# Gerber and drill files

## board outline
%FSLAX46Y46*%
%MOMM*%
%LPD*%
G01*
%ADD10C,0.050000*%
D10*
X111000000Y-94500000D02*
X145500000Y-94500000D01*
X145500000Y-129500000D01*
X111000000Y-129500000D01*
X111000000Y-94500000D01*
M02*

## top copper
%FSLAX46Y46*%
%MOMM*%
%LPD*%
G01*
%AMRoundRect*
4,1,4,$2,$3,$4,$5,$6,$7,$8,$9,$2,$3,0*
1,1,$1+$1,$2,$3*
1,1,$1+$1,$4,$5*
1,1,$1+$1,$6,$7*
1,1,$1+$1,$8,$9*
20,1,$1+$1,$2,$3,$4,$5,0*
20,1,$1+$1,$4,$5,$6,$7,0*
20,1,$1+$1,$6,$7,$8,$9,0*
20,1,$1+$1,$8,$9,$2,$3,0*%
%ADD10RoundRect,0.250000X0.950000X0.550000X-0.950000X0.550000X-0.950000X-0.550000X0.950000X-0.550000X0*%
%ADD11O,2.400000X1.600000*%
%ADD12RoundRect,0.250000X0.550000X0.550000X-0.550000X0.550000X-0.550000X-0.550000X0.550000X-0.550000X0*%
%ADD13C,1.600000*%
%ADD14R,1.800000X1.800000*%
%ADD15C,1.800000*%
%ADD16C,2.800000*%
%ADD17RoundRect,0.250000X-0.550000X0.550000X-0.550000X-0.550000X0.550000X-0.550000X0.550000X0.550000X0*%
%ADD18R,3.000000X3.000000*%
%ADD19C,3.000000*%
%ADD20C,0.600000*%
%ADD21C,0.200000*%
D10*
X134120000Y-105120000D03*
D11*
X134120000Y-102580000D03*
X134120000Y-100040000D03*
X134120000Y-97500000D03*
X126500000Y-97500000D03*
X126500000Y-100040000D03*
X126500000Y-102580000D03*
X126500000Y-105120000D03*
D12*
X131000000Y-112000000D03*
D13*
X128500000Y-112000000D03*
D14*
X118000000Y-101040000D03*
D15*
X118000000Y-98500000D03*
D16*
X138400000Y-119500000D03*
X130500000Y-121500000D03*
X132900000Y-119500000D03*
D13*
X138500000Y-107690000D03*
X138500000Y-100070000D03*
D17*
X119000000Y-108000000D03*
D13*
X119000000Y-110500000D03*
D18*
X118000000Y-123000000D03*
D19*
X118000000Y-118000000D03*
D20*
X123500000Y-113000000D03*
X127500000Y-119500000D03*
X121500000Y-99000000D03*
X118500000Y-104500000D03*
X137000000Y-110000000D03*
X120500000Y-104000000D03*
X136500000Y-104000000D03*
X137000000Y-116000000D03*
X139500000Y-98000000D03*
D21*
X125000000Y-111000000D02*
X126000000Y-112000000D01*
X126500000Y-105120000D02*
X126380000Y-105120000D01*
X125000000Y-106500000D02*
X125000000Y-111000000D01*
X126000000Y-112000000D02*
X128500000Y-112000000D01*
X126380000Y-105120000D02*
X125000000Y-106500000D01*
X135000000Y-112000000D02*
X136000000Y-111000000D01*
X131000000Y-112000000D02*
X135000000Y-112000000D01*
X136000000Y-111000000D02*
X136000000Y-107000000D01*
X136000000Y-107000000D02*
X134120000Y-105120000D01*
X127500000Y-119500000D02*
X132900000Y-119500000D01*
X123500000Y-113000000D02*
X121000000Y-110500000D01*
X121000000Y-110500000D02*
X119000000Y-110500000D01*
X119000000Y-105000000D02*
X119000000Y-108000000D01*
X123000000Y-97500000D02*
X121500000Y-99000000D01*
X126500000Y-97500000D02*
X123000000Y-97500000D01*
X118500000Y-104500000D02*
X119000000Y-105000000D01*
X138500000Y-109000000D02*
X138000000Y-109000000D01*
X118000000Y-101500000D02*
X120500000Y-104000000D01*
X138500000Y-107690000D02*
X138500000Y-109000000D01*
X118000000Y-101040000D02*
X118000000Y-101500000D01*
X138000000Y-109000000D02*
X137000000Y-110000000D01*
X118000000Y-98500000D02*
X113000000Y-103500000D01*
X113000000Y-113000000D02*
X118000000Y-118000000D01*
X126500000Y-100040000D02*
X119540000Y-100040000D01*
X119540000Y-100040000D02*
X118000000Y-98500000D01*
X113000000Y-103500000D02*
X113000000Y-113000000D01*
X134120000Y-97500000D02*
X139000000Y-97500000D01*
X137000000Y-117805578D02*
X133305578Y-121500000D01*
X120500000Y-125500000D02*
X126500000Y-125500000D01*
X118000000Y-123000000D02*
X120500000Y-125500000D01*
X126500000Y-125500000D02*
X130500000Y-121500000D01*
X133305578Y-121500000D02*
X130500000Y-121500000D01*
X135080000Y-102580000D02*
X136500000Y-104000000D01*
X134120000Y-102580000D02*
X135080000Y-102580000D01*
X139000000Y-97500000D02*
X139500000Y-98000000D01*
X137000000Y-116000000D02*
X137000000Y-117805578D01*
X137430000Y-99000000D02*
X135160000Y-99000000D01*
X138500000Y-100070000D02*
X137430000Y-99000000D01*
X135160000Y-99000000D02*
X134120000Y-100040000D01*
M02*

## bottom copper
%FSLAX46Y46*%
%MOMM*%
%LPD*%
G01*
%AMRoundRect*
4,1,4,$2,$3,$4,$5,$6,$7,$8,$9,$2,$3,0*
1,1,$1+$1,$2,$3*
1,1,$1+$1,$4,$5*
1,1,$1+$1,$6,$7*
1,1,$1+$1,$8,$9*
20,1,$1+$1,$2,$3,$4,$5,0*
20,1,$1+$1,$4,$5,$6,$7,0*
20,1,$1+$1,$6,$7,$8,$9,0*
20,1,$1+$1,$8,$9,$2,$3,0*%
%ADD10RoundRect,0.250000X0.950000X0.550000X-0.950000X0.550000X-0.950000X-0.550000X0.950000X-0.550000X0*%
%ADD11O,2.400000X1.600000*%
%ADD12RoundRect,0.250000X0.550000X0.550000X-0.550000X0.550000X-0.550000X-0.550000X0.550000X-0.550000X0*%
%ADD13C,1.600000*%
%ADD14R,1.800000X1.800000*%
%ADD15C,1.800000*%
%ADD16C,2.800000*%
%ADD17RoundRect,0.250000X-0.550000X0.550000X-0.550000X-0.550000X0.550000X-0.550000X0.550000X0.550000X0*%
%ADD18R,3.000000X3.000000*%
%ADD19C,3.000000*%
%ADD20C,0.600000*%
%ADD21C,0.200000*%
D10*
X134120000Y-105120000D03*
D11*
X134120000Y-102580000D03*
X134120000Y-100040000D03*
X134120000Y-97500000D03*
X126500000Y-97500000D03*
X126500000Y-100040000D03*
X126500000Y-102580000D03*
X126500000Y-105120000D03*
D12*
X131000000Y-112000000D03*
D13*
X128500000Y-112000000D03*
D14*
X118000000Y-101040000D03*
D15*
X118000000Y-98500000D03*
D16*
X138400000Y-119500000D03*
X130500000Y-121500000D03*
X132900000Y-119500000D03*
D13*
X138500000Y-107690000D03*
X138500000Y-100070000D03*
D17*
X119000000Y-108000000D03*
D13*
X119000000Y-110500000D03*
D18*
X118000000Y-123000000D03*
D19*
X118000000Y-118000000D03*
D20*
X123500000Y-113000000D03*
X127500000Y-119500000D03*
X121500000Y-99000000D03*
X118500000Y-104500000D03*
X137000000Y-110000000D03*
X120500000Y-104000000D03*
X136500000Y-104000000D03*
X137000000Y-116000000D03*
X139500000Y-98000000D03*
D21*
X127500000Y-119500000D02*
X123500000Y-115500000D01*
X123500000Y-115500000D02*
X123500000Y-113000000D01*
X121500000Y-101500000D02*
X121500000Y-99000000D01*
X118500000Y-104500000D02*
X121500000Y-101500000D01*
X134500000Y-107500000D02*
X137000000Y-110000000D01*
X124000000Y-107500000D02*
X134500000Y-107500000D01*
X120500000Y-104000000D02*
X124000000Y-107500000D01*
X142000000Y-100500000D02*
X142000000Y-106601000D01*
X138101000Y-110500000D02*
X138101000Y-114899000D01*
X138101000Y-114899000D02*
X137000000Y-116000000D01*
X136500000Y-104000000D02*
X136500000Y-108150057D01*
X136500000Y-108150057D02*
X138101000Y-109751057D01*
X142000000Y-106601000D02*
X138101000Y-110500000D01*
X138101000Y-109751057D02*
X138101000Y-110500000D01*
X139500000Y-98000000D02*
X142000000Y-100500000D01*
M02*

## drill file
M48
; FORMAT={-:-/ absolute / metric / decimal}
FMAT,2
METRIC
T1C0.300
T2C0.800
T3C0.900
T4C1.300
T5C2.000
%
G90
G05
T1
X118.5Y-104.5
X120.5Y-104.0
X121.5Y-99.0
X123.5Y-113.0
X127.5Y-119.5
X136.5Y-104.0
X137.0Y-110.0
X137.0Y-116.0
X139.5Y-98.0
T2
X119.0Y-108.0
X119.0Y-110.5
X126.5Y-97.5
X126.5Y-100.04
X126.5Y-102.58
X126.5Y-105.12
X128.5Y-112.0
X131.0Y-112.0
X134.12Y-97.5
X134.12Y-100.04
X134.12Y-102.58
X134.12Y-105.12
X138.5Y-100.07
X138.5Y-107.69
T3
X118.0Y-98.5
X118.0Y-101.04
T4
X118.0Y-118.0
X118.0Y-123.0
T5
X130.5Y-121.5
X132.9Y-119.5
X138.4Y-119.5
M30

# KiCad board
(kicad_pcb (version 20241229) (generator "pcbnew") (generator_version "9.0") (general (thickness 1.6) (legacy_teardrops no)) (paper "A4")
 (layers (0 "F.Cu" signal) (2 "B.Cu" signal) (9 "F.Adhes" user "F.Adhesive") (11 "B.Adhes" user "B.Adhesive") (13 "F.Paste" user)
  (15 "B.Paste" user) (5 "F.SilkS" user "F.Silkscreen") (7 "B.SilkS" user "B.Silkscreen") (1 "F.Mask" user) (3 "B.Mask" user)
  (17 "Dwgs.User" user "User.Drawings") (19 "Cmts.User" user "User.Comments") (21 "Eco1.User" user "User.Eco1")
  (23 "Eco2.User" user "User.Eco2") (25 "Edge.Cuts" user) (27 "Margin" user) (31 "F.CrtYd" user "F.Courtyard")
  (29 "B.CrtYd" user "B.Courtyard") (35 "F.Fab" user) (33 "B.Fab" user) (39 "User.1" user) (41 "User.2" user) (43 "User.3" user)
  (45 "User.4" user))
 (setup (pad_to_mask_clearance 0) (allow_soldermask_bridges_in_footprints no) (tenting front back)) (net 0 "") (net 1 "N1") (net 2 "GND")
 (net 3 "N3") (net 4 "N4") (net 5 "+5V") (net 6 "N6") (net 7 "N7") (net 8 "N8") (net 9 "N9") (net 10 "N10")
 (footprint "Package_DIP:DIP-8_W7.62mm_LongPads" (layer "F.Cu") (at 134.12 105.12 180)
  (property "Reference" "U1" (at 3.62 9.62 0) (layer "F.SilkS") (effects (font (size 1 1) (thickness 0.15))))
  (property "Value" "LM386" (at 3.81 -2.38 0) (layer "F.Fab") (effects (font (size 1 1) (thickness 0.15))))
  (pad "1" thru_hole roundrect (at 0 0 180) (size 2.4 1.6) (drill 0.8) (layers "*.Cu" "*.Mask") (remove_unused_layers no)
   (roundrect_rratio 0.15625) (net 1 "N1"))
  (pad "2" thru_hole oval (at 0 2.54 180) (size 2.4 1.6) (drill 0.8) (layers "*.Cu" "*.Mask") (remove_unused_layers no) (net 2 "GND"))
  (pad "3" thru_hole oval (at 0 5.08 180) (size 2.4 1.6) (drill 0.8) (layers "*.Cu" "*.Mask") (remove_unused_layers no) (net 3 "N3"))
  (pad "4" thru_hole oval (at 0 7.62 180) (size 2.4 1.6) (drill 0.8) (layers "*.Cu" "*.Mask") (remove_unused_layers no) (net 2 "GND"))
  (pad "5" thru_hole oval (at 7.62 7.62 180) (size 2.4 1.6) (drill 0.8) (layers "*.Cu" "*.Mask") (remove_unused_layers no) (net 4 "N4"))
  (pad "6" thru_hole oval (at 7.62 5.08 180) (size 2.4 1.6) (drill 0.8) (layers "*.Cu" "*.Mask") (remove_unused_layers no) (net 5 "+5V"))
  (pad "7" thru_hole oval (at 7.62 2.54 180) (size 2.4 1.6) (drill 0.8) (layers "*.Cu" "*.Mask") (remove_unused_layers no) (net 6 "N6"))
  (pad "8" thru_hole oval (at 7.62 0 180) (size 2.4 1.6) (drill 0.8) (layers "*.Cu" "*.Mask") (remove_unused_layers no) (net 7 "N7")))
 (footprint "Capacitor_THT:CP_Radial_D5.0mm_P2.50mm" (layer "F.Cu") (at 131 112 180)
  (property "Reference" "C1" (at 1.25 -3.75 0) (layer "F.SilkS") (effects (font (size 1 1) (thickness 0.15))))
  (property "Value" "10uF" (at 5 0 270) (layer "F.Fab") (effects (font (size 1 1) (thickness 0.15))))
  (pad "1" thru_hole roundrect (at 0 0 180) (size 1.6 1.6) (drill 0.8) (layers "*.Cu" "*.Mask") (remove_unused_layers no)
   (roundrect_rratio 0.15625) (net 1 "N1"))
  (pad "2" thru_hole circle (at 2.5 0 180) (size 1.6 1.6) (drill 0.8) (layers "*.Cu" "*.Mask") (remove_unused_layers no) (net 7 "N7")))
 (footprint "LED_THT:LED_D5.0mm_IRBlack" (layer "F.Cu") (at 118 101.04 90)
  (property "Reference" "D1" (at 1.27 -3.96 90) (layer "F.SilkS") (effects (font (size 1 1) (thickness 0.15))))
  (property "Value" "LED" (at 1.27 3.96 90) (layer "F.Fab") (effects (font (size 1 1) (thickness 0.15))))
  (pad "1" thru_hole rect (at 0 0 90) (size 1.8 1.8) (drill 0.9) (layers "*.Cu" "*.Mask") (remove_unused_layers no) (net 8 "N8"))
  (pad "2" thru_hole circle (at 2.54 0 90) (size 1.8 1.8) (drill 0.9) (layers "*.Cu" "*.Mask") (remove_unused_layers no) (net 5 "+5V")))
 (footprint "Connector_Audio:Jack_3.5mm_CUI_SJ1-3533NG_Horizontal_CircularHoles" (layer "F.Cu") (at 130.5 121.5 90)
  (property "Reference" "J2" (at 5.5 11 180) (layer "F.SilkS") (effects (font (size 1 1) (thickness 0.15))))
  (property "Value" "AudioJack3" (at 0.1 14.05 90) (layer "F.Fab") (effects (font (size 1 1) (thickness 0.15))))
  (pad "R" thru_hole circle (at 2 7.9 90) (size 2.8 2.8) (drill 2) (layers "*.Cu" "*.Mask") (remove_unused_layers no) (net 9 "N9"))
  (pad "S" thru_hole circle (at 0 0 90) (size 2.8 2.8) (drill 2) (layers "*.Cu" "*.Mask") (remove_unused_layers no) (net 2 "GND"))
  (pad "T" thru_hole circle (at 2 2.4 90) (size 2.8 2.8) (drill 2) (layers "*.Cu" "*.Mask") (remove_unused_layers no) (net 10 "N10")))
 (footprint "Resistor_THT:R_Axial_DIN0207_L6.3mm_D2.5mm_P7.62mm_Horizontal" (layer "F.Cu") (at 138.5 107.69 90)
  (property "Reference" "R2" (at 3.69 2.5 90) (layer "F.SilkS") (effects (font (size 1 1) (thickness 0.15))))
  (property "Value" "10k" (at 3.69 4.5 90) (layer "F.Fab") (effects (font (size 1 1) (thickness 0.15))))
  (pad "1" thru_hole circle (at 0 0 90) (size 1.6 1.6) (drill 0.8) (layers "*.Cu" "*.Mask") (remove_unused_layers no) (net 8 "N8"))
  (pad "2" thru_hole circle (at 7.62 0 90) (size 1.6 1.6) (drill 0.8) (layers "*.Cu" "*.Mask") (remove_unused_layers no) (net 3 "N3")))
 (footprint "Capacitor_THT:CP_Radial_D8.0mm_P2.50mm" (layer "F.Cu") (at 119 108 -90)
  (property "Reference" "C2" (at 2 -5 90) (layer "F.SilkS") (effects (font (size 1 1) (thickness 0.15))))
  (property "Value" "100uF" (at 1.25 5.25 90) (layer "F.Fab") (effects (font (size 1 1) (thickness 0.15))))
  (pad "1" thru_hole roundrect (at 0 0 270) (size 1.6 1.6) (drill 0.8) (layers "*.Cu" "*.Mask") (remove_unused_layers no)
   (roundrect_rratio 0.15625) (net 4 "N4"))
  (pad "2" thru_hole circle (at 2.5 0 270) (size 1.6 1.6) (drill 0.8) (layers "*.Cu" "*.Mask") (remove_unused_layers no) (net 10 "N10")))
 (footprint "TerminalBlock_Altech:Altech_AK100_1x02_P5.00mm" (layer "F.Cu") (at 118 123 90)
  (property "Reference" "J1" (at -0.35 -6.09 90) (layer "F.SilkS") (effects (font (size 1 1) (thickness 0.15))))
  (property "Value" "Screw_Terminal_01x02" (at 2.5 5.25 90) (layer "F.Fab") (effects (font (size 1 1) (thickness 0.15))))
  (pad "1" thru_hole rect (at 0 0 90) (size 3 3) (drill 1.3) (layers "*.Cu" "*.Mask") (remove_unused_layers no) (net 2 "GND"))
  (pad "2" thru_hole circle (at 5 0 90) (size 3 3) (drill 1.3) (layers "*.Cu" "*.Mask") (remove_unused_layers no) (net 5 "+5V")))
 (gr_rect (start 111 94.5) (end 145.5 129.5) (stroke (width 0.05) (type default)) (fill no) (layer "Edge.Cuts"))
 (segment (start 125 111) (end 126 112) (width 0.2) (layer "F.Cu") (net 7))
 (segment (start 126.5 105.12) (end 126.38 105.12) (width 0.2) (layer "F.Cu") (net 7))
 (segment (start 125 106.5) (end 125 111) (width 0.2) (layer "F.Cu") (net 7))
 (segment (start 126 112) (end 128.5 112) (width 0.2) (layer "F.Cu") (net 7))
 (segment (start 126.38 105.12) (end 125 106.5) (width 0.2) (layer "F.Cu") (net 7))
 (segment (start 135 112) (end 136 111) (width 0.2) (layer "F.Cu") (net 1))
 (segment (start 131 112) (end 135 112) (width 0.2) (layer "F.Cu") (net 1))
 (segment (start 136 111) (end 136 107) (width 0.2) (layer "F.Cu") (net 1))
 (segment (start 136 107) (end 134.12 105.12) (width 0.2) (layer "F.Cu") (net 1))
 (segment (start 127.5 119.5) (end 132.9 119.5) (width 0.2) (layer "F.Cu") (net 10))
 (segment (start 123.5 113) (end 121 110.5) (width 0.2) (layer "F.Cu") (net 10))
 (segment (start 121 110.5) (end 119 110.5) (width 0.2) (layer "F.Cu") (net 10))
 (via (at 123.5 113) (size 0.6) (drill 0.3) (layers "F.Cu" "B.Cu") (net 10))
 (via (at 127.5 119.5) (size 0.6) (drill 0.3) (layers "F.Cu" "B.Cu") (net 10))
 (segment (start 127.5 119.5) (end 123.5 115.5) (width 0.2) (layer "B.Cu") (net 10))
 (segment (start 123.5 115.5) (end 123.5 113) (width 0.2) (layer "B.Cu") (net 10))
 (segment (start 119 105) (end 119 108) (width 0.2) (layer "F.Cu") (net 4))
 (segment (start 123 97.5) (end 121.5 99) (width 0.2) (layer "F.Cu") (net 4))
 (segment (start 126.5 97.5) (end 123 97.5) (width 0.2) (layer "F.Cu") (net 4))
 (segment (start 118.5 104.5) (end 119 105) (width 0.2) (layer "F.Cu") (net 4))
 (via (at 121.5 99) (size 0.6) (drill 0.3) (layers "F.Cu" "B.Cu") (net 4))
 (via (at 118.5 104.5) (size 0.6) (drill 0.3) (layers "F.Cu" "B.Cu") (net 4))
 (segment (start 121.5 101.5) (end 121.5 99) (width 0.2) (layer "B.Cu") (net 4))
 (segment (start 118.5 104.5) (end 121.5 101.5) (width 0.2) (layer "B.Cu") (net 4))
 (segment (start 138.5 109) (end 138 109) (width 0.2) (layer "F.Cu") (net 8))
 (segment (start 118 101.5) (end 120.5 104) (width 0.2) (layer "F.Cu") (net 8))
 (segment (start 138.5 107.69) (end 138.5 109) (width 0.2) (layer "F.Cu") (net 8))
 (segment (start 118 101.04) (end 118 101.5) (width 0.2) (layer "F.Cu") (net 8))
 (segment (start 138 109) (end 137 110) (width 0.2) (layer "F.Cu") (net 8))
 (via (at 137 110) (size 0.6) (drill 0.3) (layers "F.Cu" "B.Cu") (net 8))
 (via (at 120.5 104) (size 0.6) (drill 0.3) (layers "F.Cu" "B.Cu") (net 8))
 (segment (start 134.5 107.5) (end 137 110) (width 0.2) (layer "B.Cu") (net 8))
 (segment (start 124 107.5) (end 134.5 107.5) (width 0.2) (layer "B.Cu") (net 8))
 (segment (start 120.5 104) (end 124 107.5) (width 0.2) (layer "B.Cu") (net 8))
 (segment (start 118 98.5) (end 113 103.5) (width 0.2) (layer "F.Cu") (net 5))
 (segment (start 113 113) (end 118 118) (width 0.2) (layer "F.Cu") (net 5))
 (segment (start 126.5 100.04) (end 119.54 100.04) (width 0.2) (layer "F.Cu") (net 5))
 (segment (start 119.54 100.04) (end 118 98.5) (width 0.2) (layer "F.Cu") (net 5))
 (segment (start 113 103.5) (end 113 113) (width 0.2) (layer "F.Cu") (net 5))
 (segment (start 134.12 97.5) (end 139 97.5) (width 0.2) (layer "F.Cu") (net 2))
 (segment (start 137 117.805578) (end 133.305578 121.5) (width 0.2) (layer "F.Cu") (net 2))
 (segment (start 120.5 125.5) (end 126.5 125.5) (width 0.2) (layer "F.Cu") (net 2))
 (segment (start 118 123) (end 120.5 125.5) (width 0.2) (layer "F.Cu") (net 2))
 (segment (start 126.5 125.5) (end 130.5 121.5) (width 0.2) (layer "F.Cu") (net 2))
 (segment (start 133.305578 121.5) (end 130.5 121.5) (width 0.2) (layer "F.Cu") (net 2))
 (segment (start 135.08 102.58) (end 136.5 104) (width 0.2) (layer "F.Cu") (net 2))
 (segment (start 134.12 102.58) (end 135.08 102.58) (width 0.2) (layer "F.Cu") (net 2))
 (segment (start 139 97.5) (end 139.5 98) (width 0.2) (layer "F.Cu") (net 2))
 (segment (start 137 116) (end 137 117.805578) (width 0.2) (layer "F.Cu") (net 2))
 (via (at 136.5 104) (size 0.6) (drill 0.3) (layers "F.Cu" "B.Cu") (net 2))
 (via (at 137 116) (size 0.6) (drill 0.3) (layers "F.Cu" "B.Cu") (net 2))
 (via (at 139.5 98) (size 0.6) (drill 0.3) (layers "F.Cu" "B.Cu") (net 2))
 (segment (start 142 100.5) (end 142 106.601) (width 0.2) (layer "B.Cu") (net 2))
 (segment (start 138.101 110.5) (end 138.101 114.899) (width 0.2) (layer "B.Cu") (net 2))
 (segment (start 138.101 114.899) (end 137 116) (width 0.2) (layer "B.Cu") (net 2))
 (segment (start 136.5 104) (end 136.5 108.150057) (width 0.2) (layer "B.Cu") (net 2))
 (segment (start 136.5 108.150057) (end 138.101 109.751057) (width 0.2) (layer "B.Cu") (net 2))
 (segment (start 142 106.601) (end 138.101 110.5) (width 0.2) (layer "B.Cu") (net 2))
 (segment (start 138.101 109.751057) (end 138.101 110.5) (width 0.2) (layer "B.Cu") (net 2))
 (segment (start 139.5 98) (end 142 100.5) (width 0.2) (layer "B.Cu") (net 2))
 (segment (start 137.43 99) (end 135.16 99) (width 0.2) (layer "F.Cu") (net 3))
 (segment (start 138.5 100.07) (end 137.43 99) (width 0.2) (layer "F.Cu") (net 3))
 (segment (start 135.16 99) (end 134.12 100.04) (width 0.2) (layer "F.Cu") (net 3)))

